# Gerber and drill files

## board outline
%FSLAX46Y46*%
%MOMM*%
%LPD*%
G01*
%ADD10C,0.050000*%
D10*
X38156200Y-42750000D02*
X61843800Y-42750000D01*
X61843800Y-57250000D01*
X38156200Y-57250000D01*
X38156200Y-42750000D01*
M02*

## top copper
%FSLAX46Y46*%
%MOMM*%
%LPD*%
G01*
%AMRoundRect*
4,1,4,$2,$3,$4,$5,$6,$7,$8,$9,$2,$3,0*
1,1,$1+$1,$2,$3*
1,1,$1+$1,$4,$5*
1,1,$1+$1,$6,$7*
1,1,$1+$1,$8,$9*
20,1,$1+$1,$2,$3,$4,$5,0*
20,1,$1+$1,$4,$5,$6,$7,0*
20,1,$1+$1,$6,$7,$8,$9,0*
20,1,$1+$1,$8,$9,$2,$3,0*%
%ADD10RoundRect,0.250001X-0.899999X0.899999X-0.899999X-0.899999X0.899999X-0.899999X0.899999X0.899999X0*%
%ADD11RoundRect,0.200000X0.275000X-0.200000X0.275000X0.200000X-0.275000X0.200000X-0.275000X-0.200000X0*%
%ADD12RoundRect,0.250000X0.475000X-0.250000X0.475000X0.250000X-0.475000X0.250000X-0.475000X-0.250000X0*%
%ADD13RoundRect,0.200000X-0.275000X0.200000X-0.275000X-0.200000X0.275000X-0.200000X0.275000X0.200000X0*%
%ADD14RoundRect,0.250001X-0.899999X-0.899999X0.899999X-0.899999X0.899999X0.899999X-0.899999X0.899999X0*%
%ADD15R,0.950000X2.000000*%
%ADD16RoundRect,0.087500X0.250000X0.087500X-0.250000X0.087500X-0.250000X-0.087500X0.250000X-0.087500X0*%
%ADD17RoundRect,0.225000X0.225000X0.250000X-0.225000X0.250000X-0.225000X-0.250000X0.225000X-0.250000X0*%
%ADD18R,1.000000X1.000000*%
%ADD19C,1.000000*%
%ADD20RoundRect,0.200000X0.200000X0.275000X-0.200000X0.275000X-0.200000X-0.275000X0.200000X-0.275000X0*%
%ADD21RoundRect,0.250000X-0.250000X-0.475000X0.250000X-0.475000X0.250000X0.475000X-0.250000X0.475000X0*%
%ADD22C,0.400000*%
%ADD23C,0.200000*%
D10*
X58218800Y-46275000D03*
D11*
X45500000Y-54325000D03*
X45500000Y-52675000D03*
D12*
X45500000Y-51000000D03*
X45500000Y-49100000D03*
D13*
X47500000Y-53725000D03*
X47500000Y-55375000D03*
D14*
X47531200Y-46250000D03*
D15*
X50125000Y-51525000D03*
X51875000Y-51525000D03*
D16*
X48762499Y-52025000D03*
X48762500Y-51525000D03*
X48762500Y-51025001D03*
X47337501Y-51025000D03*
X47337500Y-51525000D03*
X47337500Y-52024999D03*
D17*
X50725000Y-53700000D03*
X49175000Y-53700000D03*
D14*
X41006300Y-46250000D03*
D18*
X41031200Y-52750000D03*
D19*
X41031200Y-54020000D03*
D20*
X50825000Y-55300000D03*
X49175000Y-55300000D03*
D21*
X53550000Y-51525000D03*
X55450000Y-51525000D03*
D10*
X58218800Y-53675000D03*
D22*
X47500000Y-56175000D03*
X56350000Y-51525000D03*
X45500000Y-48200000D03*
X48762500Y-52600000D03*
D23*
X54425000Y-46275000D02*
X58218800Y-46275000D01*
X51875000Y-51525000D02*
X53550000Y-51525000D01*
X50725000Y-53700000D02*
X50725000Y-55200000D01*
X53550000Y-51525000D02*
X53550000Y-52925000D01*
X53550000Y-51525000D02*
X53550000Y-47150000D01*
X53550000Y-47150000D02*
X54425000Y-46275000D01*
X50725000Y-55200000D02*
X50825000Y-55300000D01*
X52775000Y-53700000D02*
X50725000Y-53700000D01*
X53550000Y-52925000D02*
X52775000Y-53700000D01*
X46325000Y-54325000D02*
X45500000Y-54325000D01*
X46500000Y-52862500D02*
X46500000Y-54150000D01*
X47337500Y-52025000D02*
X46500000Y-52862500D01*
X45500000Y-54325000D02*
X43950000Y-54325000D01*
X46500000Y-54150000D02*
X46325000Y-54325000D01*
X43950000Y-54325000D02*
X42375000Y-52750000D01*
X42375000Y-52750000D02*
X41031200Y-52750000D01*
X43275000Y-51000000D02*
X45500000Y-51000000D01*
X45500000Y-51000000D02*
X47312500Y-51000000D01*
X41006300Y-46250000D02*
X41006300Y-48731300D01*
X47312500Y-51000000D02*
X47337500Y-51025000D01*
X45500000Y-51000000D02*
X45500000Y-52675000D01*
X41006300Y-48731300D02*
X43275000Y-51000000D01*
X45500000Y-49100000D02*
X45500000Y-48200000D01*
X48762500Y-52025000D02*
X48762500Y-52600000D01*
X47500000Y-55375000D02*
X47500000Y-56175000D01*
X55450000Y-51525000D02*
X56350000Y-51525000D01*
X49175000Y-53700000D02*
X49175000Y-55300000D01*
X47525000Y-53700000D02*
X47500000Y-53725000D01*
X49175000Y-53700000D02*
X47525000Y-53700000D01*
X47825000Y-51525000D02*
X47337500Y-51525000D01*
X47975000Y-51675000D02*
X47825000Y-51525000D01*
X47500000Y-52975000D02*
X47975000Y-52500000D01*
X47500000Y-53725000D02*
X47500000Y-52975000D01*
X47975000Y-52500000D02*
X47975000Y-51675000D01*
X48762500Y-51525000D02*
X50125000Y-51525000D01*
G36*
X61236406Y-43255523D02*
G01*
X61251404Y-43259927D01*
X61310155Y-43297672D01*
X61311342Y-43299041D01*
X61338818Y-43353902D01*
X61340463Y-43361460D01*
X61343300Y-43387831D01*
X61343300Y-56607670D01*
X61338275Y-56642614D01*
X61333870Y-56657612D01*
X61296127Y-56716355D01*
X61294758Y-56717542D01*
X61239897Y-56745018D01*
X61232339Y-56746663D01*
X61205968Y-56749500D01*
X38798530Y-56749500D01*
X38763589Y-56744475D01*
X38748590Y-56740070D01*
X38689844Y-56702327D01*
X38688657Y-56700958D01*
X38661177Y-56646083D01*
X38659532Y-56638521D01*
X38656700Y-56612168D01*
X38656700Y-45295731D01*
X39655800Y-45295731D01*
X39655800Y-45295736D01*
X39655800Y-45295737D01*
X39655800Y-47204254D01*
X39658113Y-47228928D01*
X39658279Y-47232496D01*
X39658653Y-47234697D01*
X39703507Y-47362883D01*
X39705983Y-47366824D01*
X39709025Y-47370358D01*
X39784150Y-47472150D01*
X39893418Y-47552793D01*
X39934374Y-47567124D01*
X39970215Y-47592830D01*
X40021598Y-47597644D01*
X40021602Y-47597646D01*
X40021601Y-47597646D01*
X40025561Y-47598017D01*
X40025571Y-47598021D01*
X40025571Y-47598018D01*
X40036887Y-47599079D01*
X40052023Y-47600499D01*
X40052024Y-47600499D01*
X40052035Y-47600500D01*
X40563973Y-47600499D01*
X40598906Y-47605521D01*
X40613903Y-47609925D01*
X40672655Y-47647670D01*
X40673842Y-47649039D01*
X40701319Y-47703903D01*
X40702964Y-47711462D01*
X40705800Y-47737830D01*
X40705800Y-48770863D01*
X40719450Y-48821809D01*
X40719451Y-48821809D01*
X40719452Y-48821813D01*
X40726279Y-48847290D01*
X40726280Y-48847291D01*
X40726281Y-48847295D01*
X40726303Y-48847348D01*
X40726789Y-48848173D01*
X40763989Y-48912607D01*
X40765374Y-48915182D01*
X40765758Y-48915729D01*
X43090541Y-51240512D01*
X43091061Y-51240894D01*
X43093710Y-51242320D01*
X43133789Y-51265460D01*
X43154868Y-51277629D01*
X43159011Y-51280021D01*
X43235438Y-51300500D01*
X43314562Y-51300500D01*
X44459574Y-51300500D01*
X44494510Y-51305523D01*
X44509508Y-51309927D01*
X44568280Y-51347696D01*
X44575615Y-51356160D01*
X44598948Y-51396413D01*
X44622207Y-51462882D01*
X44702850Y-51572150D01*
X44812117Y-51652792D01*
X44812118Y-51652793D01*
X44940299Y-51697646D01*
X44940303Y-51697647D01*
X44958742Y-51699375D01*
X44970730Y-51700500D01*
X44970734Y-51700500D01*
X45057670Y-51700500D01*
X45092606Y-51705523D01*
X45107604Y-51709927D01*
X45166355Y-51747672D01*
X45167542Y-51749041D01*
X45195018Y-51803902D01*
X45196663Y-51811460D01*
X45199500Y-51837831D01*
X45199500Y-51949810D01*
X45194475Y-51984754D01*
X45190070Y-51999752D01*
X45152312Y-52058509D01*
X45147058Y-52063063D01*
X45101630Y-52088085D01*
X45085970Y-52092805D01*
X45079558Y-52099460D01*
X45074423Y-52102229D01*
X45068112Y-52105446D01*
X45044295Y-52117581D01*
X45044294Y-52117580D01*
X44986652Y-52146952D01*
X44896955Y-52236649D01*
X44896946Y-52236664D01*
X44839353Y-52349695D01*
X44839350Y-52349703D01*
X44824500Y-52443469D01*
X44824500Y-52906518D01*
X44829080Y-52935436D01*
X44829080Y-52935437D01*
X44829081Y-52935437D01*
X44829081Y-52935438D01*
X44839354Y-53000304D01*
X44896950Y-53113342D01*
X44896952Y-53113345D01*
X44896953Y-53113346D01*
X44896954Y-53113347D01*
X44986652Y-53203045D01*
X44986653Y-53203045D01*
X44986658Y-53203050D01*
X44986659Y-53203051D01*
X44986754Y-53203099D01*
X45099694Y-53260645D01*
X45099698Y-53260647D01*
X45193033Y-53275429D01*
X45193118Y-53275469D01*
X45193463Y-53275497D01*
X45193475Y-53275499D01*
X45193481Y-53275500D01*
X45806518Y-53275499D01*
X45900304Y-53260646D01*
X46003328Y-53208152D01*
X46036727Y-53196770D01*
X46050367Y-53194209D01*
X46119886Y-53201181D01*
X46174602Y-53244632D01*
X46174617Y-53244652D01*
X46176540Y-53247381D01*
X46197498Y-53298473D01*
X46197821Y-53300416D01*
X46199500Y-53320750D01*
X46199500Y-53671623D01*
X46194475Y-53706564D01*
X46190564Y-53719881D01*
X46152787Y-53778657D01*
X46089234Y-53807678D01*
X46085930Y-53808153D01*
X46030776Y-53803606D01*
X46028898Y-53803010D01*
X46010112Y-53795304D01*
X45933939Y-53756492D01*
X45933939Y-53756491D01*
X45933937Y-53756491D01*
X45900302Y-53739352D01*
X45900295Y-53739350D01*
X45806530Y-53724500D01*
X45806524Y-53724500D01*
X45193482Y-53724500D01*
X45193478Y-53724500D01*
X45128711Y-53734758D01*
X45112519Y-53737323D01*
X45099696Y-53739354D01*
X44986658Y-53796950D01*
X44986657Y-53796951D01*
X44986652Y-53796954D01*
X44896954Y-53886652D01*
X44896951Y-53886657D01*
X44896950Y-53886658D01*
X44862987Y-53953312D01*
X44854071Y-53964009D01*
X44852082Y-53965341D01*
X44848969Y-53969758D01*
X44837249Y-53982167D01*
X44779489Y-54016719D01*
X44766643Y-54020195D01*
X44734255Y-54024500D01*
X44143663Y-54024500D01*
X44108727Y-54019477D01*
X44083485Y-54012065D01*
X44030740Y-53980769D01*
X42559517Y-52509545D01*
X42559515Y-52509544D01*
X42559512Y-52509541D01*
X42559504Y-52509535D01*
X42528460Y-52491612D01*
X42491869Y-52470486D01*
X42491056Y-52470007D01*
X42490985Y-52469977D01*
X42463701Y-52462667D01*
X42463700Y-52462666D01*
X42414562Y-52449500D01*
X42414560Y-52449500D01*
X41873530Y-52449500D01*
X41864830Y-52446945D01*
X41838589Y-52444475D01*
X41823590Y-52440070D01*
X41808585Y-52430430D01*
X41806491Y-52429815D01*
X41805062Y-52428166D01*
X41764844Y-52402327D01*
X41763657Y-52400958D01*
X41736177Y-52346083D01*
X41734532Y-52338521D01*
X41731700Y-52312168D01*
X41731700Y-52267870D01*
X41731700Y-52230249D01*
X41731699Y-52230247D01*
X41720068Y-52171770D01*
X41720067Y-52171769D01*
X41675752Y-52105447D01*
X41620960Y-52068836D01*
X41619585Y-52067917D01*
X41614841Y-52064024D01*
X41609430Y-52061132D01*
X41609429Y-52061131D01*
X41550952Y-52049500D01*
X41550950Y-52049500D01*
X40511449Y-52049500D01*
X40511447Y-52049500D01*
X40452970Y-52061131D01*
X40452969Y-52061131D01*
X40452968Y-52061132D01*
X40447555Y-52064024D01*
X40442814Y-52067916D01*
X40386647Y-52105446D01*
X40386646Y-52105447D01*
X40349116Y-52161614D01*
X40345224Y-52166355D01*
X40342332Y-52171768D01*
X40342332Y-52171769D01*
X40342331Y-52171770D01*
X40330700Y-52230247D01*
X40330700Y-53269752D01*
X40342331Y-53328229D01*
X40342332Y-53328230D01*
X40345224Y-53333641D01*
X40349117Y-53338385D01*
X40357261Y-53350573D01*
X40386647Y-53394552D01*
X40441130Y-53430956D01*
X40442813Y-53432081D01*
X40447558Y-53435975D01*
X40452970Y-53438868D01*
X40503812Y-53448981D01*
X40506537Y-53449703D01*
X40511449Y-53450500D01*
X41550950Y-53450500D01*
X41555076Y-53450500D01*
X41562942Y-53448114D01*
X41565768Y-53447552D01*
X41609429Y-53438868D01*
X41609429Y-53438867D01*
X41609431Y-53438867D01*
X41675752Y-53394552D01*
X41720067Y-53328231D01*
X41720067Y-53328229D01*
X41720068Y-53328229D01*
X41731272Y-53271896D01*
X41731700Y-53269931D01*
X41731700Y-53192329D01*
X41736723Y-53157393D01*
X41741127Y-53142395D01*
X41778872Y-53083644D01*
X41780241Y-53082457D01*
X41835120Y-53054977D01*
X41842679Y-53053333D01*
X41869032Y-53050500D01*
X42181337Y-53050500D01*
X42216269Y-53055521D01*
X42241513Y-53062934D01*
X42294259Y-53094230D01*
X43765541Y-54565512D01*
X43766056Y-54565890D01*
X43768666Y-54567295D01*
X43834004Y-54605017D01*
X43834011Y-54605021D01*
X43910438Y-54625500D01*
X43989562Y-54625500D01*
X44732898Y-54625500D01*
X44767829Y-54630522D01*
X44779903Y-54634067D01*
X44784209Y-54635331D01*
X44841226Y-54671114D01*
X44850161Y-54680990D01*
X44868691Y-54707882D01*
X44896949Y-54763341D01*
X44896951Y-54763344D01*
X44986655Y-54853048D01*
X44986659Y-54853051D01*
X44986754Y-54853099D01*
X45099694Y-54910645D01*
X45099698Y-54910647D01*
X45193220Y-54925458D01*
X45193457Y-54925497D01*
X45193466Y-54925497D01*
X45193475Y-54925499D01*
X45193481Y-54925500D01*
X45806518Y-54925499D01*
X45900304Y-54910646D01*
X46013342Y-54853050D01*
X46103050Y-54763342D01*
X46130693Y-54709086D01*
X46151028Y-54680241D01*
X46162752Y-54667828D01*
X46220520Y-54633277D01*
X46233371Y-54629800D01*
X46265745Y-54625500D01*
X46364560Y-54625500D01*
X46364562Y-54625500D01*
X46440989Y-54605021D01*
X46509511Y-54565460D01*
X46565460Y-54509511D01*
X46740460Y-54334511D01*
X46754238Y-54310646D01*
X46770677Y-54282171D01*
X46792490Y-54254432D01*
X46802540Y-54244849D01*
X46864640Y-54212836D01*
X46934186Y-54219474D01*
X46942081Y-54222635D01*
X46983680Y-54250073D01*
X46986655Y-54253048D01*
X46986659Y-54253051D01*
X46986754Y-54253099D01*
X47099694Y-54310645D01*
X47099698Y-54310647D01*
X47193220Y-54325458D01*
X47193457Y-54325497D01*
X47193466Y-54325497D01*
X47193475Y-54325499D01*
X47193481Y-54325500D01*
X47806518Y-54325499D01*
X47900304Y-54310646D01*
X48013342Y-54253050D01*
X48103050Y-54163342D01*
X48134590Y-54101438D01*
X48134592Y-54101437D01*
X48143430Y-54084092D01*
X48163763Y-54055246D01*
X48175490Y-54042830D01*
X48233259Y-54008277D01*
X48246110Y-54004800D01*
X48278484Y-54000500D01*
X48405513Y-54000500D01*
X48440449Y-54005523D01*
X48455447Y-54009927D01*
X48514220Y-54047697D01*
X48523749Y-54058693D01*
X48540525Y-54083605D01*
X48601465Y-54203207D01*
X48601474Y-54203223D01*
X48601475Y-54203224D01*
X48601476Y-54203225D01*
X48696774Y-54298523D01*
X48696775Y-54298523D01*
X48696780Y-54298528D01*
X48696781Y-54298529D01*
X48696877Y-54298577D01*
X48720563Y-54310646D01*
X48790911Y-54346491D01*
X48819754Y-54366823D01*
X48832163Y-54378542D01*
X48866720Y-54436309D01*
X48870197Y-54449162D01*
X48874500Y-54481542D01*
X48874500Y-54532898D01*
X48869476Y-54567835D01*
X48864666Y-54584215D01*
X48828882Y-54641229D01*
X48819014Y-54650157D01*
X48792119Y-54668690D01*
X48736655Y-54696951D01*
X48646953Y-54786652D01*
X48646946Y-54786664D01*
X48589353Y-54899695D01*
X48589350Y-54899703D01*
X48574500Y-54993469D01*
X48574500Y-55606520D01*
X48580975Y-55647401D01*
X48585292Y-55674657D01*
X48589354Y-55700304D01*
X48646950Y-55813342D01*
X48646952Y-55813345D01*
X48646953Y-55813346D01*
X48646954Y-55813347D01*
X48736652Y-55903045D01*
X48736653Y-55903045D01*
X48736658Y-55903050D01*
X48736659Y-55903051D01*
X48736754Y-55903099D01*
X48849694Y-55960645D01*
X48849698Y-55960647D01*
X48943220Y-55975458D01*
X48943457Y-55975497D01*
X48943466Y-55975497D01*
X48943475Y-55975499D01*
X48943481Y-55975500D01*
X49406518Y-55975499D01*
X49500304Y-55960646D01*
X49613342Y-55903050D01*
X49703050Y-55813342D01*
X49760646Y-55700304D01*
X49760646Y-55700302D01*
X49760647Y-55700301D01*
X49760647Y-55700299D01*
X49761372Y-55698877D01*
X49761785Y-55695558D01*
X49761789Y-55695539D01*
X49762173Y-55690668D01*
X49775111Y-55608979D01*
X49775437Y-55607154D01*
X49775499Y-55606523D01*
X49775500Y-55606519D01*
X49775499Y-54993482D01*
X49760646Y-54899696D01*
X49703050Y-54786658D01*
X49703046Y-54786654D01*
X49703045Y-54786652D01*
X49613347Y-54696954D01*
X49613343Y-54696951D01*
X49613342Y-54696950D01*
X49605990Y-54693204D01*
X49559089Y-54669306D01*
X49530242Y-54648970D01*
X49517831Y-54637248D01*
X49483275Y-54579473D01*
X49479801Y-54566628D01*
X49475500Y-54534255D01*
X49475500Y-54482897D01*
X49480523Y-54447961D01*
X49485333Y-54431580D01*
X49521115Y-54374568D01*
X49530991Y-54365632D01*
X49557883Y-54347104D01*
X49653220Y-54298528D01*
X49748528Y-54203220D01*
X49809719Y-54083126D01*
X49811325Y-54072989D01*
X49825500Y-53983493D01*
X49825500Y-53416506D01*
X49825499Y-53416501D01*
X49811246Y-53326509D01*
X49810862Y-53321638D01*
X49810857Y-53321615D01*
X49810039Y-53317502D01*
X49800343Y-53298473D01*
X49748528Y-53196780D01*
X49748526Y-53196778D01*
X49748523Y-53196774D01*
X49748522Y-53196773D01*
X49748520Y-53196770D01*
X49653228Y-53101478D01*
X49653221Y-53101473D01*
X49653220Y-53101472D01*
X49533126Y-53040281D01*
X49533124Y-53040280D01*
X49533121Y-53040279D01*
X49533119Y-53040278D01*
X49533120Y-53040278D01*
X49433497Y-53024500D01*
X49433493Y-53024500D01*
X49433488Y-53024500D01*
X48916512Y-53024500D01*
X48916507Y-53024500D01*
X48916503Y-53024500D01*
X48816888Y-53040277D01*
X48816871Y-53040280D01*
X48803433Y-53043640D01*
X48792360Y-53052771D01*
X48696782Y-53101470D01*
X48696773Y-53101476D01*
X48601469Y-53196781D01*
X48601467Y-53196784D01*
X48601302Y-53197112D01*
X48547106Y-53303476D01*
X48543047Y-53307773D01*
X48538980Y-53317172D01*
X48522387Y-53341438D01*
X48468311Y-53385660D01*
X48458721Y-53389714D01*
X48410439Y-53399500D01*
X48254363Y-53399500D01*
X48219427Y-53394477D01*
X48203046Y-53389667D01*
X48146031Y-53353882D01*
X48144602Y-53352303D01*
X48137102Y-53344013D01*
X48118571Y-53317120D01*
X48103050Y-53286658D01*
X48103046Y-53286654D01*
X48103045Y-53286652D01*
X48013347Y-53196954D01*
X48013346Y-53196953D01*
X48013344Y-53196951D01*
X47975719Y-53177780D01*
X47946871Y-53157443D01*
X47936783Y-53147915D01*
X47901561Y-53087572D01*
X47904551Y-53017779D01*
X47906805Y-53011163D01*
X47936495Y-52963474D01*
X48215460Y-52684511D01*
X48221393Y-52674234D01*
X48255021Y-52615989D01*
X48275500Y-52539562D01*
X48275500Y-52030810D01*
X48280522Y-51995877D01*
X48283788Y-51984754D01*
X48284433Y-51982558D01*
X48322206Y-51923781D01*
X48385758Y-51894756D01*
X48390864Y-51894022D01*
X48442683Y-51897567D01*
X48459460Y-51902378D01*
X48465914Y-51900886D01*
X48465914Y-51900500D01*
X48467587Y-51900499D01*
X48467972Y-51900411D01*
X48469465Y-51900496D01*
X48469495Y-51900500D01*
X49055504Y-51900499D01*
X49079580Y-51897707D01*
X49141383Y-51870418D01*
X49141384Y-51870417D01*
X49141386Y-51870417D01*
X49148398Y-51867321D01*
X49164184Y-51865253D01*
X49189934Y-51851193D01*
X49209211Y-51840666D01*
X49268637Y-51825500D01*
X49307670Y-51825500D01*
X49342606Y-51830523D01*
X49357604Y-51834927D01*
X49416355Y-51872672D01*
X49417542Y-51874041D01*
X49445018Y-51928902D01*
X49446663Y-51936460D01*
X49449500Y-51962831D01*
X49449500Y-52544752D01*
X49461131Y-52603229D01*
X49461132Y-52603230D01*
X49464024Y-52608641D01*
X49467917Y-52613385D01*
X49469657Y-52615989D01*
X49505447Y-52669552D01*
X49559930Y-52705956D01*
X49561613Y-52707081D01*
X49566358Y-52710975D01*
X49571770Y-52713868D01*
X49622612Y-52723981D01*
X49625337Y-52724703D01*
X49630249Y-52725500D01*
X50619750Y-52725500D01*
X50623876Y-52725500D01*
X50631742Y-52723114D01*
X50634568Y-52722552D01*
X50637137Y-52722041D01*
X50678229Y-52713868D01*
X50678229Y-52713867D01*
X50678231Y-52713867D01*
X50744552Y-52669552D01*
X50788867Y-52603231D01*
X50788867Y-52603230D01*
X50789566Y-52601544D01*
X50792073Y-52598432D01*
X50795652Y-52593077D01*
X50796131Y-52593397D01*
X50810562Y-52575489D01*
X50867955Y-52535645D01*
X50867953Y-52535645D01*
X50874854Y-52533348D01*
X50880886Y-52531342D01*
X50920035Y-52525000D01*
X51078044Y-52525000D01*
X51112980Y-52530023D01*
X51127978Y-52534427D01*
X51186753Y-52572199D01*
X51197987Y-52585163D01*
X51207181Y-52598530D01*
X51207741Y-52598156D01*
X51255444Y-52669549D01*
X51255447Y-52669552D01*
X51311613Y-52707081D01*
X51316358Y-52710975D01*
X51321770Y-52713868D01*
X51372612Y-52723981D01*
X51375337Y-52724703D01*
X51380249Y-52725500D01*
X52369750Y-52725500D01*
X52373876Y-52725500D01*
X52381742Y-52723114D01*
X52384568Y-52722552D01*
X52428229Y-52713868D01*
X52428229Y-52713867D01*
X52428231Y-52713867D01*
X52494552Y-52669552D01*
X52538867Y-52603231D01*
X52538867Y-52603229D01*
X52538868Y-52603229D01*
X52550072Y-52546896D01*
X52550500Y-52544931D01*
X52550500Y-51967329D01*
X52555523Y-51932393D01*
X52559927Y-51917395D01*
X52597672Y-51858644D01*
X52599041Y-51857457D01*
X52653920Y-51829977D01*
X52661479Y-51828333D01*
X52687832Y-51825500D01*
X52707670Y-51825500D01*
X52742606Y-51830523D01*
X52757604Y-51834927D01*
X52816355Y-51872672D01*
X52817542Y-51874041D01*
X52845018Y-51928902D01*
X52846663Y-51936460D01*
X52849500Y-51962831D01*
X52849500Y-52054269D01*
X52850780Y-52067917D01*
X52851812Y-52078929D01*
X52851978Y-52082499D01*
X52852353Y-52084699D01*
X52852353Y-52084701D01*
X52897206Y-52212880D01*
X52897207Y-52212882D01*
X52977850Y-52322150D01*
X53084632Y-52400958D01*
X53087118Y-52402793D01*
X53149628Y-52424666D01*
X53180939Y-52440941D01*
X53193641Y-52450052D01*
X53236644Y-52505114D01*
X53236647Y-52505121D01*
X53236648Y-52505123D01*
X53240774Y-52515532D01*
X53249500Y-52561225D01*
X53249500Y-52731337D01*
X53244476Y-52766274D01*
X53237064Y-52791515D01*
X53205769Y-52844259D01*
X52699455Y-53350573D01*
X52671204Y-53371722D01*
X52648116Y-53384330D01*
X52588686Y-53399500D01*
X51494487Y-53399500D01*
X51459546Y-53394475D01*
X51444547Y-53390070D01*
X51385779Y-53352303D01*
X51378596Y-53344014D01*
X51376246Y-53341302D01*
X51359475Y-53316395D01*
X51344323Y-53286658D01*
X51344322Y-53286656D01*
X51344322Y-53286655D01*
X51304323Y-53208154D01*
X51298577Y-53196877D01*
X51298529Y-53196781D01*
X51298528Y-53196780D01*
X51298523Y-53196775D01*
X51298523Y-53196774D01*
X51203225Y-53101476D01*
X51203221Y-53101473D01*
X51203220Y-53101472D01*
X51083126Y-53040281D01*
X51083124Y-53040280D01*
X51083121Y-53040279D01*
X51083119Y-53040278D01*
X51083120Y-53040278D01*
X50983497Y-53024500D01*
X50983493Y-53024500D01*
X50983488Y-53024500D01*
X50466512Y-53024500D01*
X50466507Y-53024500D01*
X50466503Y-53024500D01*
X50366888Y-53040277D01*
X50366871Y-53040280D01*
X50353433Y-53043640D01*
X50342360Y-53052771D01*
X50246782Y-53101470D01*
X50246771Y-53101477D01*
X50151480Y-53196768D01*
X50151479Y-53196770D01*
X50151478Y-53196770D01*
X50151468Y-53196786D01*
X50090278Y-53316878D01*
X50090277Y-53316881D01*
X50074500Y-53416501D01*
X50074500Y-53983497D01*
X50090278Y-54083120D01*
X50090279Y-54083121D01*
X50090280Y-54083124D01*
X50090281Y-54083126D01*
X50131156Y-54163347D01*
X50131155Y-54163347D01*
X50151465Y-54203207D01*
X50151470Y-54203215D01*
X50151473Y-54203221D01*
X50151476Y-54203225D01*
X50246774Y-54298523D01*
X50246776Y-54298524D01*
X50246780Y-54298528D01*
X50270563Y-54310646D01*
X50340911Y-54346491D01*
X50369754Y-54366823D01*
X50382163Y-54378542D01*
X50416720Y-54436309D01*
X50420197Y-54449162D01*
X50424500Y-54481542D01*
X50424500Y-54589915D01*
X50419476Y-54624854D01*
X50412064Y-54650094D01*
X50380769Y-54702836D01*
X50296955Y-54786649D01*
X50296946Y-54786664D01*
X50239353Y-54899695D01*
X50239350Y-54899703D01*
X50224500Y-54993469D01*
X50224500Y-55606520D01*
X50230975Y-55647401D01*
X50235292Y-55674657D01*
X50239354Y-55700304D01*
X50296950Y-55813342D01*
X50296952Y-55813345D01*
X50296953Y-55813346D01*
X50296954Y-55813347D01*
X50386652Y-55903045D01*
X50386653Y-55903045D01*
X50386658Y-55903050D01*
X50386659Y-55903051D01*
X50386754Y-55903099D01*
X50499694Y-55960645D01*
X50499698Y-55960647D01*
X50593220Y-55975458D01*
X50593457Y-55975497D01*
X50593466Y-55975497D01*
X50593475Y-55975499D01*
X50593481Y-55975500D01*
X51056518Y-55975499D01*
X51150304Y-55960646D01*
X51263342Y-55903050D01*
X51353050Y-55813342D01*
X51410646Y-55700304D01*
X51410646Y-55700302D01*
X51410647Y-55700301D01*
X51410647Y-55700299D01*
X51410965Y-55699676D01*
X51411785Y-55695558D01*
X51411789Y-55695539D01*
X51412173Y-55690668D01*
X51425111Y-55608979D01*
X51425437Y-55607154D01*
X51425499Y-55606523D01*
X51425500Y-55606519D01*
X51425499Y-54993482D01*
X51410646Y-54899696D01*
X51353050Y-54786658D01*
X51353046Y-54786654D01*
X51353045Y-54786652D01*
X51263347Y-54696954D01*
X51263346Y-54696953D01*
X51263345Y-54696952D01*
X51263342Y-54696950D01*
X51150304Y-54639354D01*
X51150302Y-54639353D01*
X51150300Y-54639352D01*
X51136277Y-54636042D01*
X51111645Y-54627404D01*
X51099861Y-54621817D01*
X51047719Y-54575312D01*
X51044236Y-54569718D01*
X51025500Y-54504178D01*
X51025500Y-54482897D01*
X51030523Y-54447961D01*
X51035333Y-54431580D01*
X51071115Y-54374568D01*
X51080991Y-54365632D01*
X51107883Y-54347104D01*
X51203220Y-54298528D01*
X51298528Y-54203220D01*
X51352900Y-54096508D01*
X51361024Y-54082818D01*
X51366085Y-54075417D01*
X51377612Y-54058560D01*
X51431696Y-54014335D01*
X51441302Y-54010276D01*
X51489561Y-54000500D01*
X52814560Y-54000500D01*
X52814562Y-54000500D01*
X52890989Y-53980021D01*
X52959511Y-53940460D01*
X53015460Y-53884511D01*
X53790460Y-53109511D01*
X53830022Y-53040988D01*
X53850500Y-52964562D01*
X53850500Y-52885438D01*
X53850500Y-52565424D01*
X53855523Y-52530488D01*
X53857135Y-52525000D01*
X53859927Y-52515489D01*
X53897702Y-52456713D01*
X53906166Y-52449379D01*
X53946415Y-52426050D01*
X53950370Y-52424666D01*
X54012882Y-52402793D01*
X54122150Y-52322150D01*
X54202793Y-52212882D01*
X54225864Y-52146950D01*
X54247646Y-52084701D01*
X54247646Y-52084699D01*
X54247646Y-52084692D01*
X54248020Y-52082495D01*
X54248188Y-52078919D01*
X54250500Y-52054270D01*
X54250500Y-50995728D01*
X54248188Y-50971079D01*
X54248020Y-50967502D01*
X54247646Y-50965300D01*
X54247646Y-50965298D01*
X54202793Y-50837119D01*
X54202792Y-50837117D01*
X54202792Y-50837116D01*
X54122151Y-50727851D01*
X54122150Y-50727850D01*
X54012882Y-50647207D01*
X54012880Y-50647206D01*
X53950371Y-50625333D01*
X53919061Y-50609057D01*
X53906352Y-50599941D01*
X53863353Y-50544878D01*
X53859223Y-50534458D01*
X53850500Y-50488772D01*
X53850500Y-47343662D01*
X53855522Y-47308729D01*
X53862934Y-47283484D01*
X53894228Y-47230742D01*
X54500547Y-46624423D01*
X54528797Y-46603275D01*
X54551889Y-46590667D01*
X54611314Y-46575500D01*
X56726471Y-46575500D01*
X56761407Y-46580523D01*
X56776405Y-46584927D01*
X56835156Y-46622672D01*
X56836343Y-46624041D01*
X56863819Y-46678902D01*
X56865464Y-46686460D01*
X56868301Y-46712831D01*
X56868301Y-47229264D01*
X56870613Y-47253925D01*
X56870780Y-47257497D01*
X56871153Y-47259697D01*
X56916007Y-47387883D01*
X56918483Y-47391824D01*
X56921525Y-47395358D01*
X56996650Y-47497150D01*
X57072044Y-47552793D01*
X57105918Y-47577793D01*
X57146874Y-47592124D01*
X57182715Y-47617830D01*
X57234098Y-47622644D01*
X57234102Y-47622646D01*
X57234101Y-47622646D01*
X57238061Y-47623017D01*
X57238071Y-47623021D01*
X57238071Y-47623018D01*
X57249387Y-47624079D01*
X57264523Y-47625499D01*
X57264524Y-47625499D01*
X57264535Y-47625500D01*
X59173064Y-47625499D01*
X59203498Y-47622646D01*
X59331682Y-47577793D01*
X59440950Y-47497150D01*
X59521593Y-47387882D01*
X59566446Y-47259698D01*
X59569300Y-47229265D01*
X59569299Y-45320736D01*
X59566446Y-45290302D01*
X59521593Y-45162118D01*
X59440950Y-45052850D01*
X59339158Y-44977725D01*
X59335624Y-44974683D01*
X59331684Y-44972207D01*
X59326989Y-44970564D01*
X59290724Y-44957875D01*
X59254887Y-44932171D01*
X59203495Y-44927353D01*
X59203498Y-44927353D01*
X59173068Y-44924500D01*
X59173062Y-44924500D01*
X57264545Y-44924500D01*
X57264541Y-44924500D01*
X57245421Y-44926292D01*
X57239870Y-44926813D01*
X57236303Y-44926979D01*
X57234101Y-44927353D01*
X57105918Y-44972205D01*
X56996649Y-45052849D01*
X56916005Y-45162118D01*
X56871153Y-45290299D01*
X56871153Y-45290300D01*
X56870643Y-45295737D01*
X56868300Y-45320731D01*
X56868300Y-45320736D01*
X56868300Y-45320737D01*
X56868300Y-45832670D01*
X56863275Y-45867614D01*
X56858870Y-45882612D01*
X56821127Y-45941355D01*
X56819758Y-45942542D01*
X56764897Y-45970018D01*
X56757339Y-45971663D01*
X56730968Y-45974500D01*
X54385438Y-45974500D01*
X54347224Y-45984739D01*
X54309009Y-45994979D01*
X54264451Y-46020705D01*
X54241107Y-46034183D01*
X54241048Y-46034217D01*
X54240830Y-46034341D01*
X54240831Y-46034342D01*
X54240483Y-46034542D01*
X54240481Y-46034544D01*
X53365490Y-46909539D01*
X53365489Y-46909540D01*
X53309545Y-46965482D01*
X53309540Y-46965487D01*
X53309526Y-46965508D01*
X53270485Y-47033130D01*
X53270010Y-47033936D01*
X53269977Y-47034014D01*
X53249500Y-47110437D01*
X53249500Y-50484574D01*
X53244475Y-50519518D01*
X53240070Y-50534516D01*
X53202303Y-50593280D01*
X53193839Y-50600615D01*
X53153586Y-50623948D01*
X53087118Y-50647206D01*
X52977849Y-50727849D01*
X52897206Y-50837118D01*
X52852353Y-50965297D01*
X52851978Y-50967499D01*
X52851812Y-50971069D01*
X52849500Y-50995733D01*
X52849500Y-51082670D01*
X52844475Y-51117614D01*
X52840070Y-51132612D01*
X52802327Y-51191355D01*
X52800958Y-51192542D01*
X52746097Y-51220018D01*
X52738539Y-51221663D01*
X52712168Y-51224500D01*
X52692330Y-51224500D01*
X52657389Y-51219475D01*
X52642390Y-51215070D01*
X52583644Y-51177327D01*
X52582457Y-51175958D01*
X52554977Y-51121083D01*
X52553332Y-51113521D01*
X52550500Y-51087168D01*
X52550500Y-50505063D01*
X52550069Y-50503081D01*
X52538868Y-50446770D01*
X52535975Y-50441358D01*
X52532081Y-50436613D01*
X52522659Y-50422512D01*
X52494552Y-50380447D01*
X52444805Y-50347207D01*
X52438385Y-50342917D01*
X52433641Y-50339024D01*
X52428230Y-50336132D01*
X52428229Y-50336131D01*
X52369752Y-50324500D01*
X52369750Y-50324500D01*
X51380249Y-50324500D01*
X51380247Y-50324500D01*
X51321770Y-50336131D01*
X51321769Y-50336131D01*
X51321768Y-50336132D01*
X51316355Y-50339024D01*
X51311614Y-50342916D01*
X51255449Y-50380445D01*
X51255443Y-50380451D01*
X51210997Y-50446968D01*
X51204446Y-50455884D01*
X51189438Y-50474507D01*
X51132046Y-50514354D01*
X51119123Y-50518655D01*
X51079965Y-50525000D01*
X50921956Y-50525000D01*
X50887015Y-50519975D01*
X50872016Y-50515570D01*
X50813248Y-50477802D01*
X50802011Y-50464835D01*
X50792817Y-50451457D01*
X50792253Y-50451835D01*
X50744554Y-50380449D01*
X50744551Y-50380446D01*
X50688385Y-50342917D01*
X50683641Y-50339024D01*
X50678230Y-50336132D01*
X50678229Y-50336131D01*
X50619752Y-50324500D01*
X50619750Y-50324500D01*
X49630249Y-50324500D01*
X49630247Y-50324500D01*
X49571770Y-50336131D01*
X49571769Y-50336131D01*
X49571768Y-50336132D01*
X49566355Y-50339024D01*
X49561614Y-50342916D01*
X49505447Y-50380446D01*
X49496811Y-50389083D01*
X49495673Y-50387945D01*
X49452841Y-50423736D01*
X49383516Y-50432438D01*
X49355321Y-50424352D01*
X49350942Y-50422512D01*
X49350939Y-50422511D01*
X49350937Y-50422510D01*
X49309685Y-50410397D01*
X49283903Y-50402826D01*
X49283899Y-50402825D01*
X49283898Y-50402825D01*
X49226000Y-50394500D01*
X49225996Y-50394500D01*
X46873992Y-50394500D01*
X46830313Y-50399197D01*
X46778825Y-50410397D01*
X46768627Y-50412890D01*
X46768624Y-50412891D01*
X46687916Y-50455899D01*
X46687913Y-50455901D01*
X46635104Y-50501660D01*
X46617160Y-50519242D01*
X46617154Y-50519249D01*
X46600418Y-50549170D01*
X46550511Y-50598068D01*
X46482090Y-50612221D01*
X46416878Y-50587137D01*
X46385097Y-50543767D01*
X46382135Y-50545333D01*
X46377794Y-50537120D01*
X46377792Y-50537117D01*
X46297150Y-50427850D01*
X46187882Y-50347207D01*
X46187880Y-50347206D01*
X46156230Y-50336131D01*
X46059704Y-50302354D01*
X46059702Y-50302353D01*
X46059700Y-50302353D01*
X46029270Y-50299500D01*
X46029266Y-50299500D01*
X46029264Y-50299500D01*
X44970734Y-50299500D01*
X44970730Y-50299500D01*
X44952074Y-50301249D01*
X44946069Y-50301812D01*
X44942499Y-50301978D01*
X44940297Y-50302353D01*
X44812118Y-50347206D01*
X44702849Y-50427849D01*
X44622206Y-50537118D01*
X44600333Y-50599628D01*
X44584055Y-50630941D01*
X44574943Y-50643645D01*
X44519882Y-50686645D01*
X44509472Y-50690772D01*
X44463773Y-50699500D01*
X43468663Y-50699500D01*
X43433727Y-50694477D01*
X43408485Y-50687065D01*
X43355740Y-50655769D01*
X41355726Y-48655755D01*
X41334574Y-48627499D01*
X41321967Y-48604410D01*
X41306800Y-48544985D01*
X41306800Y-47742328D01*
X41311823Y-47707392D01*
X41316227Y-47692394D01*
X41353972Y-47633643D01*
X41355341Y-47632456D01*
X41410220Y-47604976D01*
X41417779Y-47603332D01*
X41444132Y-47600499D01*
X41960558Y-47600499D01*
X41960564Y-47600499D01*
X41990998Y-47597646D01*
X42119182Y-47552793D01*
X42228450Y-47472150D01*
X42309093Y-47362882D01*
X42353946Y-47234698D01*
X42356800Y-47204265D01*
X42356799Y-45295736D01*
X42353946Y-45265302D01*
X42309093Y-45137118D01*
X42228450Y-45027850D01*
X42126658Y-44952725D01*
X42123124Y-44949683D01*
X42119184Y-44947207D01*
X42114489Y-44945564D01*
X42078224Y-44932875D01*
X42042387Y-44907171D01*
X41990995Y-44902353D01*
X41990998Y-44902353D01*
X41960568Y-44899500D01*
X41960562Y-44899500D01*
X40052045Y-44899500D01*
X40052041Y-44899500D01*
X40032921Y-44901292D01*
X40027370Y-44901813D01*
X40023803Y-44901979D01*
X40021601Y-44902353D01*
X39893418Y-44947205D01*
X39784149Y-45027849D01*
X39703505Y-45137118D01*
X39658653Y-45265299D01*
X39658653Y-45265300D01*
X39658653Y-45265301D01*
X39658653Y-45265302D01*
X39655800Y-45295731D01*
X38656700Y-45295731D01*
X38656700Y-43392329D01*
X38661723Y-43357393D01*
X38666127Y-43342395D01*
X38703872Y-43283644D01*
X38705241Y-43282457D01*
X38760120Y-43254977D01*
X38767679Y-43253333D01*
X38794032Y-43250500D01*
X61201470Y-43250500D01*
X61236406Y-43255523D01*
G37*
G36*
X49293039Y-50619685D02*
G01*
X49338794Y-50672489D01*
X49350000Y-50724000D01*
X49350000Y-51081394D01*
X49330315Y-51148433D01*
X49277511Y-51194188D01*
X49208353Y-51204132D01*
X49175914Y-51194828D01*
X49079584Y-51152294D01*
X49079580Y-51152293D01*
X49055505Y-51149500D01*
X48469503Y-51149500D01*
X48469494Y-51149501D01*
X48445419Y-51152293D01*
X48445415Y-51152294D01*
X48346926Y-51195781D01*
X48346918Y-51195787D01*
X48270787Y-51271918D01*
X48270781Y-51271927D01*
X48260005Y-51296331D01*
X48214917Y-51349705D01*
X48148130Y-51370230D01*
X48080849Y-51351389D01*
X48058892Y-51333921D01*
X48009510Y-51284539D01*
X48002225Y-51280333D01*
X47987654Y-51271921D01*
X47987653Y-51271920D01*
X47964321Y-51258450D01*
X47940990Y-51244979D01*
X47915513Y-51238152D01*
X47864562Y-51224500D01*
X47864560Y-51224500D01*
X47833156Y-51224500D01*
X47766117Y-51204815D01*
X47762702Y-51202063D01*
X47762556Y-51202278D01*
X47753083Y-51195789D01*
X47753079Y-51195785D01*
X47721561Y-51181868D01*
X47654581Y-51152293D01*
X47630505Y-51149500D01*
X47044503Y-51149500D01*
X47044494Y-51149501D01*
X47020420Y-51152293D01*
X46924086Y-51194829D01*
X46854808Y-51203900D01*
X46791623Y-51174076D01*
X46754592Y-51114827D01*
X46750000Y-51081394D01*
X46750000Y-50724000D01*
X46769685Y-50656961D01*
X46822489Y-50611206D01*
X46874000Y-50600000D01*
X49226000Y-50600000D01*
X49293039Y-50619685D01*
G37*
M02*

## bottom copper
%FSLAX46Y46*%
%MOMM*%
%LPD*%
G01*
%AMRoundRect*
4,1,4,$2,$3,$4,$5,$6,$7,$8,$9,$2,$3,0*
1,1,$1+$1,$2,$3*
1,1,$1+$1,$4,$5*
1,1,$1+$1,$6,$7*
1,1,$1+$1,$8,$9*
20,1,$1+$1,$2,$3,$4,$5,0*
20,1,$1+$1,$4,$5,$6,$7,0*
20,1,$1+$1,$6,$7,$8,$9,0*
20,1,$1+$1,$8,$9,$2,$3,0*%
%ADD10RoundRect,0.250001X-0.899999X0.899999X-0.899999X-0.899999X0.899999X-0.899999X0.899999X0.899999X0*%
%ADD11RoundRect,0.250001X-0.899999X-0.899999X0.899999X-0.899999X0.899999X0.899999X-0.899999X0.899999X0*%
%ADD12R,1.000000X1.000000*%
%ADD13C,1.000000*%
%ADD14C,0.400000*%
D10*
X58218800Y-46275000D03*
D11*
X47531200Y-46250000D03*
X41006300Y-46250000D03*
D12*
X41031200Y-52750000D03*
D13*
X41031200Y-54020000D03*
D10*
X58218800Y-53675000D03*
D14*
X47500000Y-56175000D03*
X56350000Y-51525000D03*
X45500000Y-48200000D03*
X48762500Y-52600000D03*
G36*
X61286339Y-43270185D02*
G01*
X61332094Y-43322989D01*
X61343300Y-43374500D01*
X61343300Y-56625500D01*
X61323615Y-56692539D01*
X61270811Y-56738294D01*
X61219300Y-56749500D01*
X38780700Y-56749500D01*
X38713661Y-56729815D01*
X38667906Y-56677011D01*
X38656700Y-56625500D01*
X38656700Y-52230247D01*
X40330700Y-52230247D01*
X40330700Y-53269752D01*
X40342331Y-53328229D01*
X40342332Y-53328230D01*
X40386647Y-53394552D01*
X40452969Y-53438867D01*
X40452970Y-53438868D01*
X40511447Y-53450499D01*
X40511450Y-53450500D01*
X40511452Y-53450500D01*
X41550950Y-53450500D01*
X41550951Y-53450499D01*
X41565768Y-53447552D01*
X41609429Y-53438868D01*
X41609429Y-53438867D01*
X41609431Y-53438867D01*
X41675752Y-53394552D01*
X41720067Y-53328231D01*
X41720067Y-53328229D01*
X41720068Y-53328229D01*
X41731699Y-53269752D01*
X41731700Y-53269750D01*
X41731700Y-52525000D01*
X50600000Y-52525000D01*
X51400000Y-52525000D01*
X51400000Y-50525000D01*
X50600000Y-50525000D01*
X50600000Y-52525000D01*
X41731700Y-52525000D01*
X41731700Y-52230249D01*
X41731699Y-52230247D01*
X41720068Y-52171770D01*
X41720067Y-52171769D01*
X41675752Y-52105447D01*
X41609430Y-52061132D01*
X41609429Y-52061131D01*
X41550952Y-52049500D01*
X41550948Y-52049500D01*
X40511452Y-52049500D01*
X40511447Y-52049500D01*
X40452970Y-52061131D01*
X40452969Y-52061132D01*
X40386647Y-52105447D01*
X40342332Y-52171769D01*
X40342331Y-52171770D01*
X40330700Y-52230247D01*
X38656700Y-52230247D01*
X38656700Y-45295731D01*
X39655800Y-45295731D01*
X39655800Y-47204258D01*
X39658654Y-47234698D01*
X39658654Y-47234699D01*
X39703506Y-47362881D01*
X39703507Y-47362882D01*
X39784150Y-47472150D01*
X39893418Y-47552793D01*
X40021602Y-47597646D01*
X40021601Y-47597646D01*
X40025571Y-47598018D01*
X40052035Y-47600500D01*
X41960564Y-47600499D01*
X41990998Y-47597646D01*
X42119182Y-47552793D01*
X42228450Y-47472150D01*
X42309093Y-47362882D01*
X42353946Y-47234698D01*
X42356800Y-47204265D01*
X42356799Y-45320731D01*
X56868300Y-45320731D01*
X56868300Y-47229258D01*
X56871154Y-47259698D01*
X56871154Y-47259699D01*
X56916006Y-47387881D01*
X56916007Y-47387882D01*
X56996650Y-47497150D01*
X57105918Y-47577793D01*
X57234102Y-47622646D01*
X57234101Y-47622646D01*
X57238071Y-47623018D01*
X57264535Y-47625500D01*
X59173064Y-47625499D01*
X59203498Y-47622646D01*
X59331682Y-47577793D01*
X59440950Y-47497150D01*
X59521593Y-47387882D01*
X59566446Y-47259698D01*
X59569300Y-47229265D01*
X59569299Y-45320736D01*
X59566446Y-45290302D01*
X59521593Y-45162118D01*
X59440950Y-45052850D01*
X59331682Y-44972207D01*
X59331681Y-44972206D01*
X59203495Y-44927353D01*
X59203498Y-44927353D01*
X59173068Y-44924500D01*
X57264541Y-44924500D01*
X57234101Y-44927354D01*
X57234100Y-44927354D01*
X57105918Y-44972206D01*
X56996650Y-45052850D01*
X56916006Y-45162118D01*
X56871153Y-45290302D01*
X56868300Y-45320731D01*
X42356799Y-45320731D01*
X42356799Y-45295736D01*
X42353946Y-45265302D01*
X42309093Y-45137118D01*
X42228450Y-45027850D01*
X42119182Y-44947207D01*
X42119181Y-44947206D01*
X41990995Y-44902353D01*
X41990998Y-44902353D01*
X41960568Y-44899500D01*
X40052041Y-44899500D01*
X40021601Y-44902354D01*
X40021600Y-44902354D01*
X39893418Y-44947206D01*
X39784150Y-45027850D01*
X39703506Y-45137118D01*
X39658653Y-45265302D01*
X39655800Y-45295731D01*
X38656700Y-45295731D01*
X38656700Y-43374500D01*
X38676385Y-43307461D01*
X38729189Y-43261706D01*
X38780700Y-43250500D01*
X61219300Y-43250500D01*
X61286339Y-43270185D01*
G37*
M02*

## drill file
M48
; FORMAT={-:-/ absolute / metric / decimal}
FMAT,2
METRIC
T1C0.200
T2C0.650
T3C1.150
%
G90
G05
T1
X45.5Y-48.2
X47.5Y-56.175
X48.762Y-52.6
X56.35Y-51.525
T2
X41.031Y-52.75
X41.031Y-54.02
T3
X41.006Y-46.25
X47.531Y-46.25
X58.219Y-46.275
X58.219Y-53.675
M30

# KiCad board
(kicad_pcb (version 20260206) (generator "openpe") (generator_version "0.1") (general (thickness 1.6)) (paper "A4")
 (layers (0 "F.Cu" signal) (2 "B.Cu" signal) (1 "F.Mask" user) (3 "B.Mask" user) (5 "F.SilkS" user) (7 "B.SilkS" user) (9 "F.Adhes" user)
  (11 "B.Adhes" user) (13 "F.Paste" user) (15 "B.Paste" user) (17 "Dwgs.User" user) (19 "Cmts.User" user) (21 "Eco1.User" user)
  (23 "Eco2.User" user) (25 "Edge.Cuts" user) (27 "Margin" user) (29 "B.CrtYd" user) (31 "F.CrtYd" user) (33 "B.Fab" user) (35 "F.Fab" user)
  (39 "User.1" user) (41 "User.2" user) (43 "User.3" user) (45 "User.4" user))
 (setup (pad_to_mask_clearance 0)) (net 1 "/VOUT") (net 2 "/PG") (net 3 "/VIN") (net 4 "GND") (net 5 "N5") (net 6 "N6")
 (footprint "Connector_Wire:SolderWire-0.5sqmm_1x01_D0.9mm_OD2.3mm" (layer "F.Cu") (at 58.2188 46.275 -90)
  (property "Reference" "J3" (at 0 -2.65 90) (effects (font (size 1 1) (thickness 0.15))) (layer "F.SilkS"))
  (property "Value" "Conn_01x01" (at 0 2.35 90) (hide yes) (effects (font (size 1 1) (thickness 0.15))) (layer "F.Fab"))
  (pad "1" thru_hole roundrect (at 0 0 -90) (size 2.3 2.3) (drill 1.15) (layers "*.Cu" "*.Mask") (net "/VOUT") (roundrect_rratio 0.108696)
   (remove_unused_layers no)))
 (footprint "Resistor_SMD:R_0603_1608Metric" (layer "F.Cu") (at 45.5 53.5 90)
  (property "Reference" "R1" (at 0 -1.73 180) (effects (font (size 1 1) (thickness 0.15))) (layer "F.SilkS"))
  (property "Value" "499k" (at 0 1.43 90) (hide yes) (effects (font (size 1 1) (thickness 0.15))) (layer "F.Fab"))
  (pad "1" smd roundrect (at -0.825 0 90) (size 0.8 0.95) (layers "F.Cu" "F.Mask" "F.Paste") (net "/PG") (roundrect_rratio 0.25))
  (pad "2" smd roundrect (at 0.825 0 90) (size 0.8 0.95) (layers "F.Cu" "F.Mask" "F.Paste") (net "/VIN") (roundrect_rratio 0.25)))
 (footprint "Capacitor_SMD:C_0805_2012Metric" (layer "F.Cu") (at 45.5 50.05 90)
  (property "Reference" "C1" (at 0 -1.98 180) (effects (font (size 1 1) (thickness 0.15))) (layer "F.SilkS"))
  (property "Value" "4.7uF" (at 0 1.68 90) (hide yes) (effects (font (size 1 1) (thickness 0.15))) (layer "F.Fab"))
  (pad "1" smd roundrect (at -0.95 0 90) (size 1 1.45) (layers "F.Cu" "F.Mask" "F.Paste") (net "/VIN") (roundrect_rratio 0.25))
  (pad "2" smd roundrect (at 0.95 0 90) (size 1 1.45) (layers "F.Cu" "F.Mask" "F.Paste") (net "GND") (roundrect_rratio 0.25)))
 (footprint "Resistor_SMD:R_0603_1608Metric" (layer "F.Cu") (at 47.5 54.55 -90)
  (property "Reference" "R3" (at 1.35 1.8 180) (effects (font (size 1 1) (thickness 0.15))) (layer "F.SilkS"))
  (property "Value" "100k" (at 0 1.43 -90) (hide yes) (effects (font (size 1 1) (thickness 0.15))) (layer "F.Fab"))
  (pad "1" smd roundrect (at -0.825 0 -90) (size 0.8 0.95) (layers "F.Cu" "F.Mask" "F.Paste") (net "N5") (roundrect_rratio 0.25))
  (pad "2" smd roundrect (at 0.825 0 -90) (size 0.8 0.95) (layers "F.Cu" "F.Mask" "F.Paste") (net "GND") (roundrect_rratio 0.25)))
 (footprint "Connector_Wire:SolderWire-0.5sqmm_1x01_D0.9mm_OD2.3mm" (layer "F.Cu") (at 47.5312 46.25 0)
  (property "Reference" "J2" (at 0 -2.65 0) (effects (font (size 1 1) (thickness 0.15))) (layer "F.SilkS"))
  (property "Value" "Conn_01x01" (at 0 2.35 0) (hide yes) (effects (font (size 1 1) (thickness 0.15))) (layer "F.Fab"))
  (pad "1" thru_hole roundrect (at 0 0 0) (size 2.3 2.3) (drill 1.15) (layers "*.Cu" "*.Mask") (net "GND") (roundrect_rratio 0.108696)
   (remove_unused_layers no)))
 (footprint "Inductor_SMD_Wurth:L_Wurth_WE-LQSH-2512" (layer "F.Cu") (at 51 51.525 0)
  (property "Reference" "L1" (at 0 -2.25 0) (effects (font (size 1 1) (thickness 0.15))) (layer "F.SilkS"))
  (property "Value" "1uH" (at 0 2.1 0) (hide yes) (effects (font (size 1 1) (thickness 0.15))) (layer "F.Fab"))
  (pad "1" smd rect (at -0.875 0 0) (size 0.95 2) (layers "F.Cu" "F.Mask" "F.Paste") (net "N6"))
  (pad "2" smd rect (at 0.875 0 0) (size 0.95 2) (layers "F.Cu" "F.Mask" "F.Paste") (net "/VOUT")))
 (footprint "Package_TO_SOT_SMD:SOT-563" (layer "F.Cu") (at 48.05 51.525 180)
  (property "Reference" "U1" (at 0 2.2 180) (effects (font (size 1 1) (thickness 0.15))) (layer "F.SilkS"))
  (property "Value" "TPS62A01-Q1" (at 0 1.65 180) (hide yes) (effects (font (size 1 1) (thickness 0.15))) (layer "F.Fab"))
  (pad "1" smd roundrect (at -0.712499 -0.5 180) (size 0.675 0.35) (layers "F.Cu" "F.Mask" "F.Paste") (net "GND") (roundrect_rratio 0.25))
  (pad "2" smd roundrect (at -0.7125 0 180) (size 0.675 0.35) (layers "F.Cu" "F.Mask" "F.Paste") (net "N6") (roundrect_rratio 0.25))
  (pad "3" smd roundrect (at -0.7125 0.499999 180) (size 0.675 0.35) (layers "F.Cu" "F.Mask" "F.Paste") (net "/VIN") (roundrect_rratio 0.25))
  (pad "4" smd roundrect (at 0.712499 0.5 180) (size 0.675 0.35) (layers "F.Cu" "F.Mask" "F.Paste") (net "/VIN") (roundrect_rratio 0.25))
  (pad "5" smd roundrect (at 0.7125 0 180) (size 0.675 0.35) (layers "F.Cu" "F.Mask" "F.Paste") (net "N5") (roundrect_rratio 0.25))
  (pad "6" smd roundrect (at 0.7125 -0.499999 180) (size 0.675 0.35) (layers "F.Cu" "F.Mask" "F.Paste") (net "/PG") (roundrect_rratio 0.25)))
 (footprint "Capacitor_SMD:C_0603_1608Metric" (layer "F.Cu") (at 49.95 53.7 180)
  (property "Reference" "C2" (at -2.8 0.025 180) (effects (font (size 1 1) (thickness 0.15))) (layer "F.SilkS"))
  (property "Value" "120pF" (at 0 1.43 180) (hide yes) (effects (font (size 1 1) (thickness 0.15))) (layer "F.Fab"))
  (pad "1" smd roundrect (at -0.775 0 180) (size 0.9 0.95) (layers "F.Cu" "F.Mask" "F.Paste") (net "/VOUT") (roundrect_rratio 0.25))
  (pad "2" smd roundrect (at 0.775 0 180) (size 0.9 0.95) (layers "F.Cu" "F.Mask" "F.Paste") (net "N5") (roundrect_rratio 0.25)))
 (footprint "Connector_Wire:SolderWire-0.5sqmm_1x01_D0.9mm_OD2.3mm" (layer "F.Cu") (at 41.0063 46.25 0)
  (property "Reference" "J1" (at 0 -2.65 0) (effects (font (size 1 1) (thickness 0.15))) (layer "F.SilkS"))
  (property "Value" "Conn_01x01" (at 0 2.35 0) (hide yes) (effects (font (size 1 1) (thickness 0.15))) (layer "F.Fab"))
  (pad "1" thru_hole roundrect (at 0 0 0) (size 2.3 2.3) (drill 1.15) (layers "*.Cu" "*.Mask") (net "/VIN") (roundrect_rratio 0.108696)
   (remove_unused_layers no)))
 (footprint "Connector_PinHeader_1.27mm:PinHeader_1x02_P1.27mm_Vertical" (layer "F.Cu") (at 41.0312 53.385 0)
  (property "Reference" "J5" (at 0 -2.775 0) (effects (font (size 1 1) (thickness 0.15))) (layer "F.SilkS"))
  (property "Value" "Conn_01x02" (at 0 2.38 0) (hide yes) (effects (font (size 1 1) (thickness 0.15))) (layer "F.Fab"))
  (pad "1" thru_hole rect (at 0 -0.635 0) (size 1 1) (drill 0.65) (layers "*.Cu" "*.Mask") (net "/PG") (remove_unused_layers no))
  (pad "2" thru_hole circle (at 0 0.635 0) (size 1 1) (drill 0.65) (layers "*.Cu" "*.Mask") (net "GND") (remove_unused_layers no)))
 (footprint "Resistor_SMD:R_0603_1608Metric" (layer "F.Cu") (at 50 55.3 180)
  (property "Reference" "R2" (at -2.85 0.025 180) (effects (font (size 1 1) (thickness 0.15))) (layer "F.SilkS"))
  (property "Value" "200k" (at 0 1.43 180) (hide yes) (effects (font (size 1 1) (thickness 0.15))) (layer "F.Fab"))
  (pad "1" smd roundrect (at -0.825 0 180) (size 0.8 0.95) (layers "F.Cu" "F.Mask" "F.Paste") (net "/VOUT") (roundrect_rratio 0.25))
  (pad "2" smd roundrect (at 0.825 0 180) (size 0.8 0.95) (layers "F.Cu" "F.Mask" "F.Paste") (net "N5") (roundrect_rratio 0.25)))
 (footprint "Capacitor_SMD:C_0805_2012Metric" (layer "F.Cu") (at 54.5 51.525 0)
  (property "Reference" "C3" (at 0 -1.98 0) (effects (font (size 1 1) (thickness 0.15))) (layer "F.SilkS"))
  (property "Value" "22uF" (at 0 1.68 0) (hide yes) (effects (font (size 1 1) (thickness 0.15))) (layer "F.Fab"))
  (pad "1" smd roundrect (at -0.95 0 0) (size 1 1.45) (layers "F.Cu" "F.Mask" "F.Paste") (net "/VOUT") (roundrect_rratio 0.25))
  (pad "2" smd roundrect (at 0.95 0 0) (size 1 1.45) (layers "F.Cu" "F.Mask" "F.Paste") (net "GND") (roundrect_rratio 0.25)))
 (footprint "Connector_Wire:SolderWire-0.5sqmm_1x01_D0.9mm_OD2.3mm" (layer "F.Cu") (at 58.2188 53.675 -90)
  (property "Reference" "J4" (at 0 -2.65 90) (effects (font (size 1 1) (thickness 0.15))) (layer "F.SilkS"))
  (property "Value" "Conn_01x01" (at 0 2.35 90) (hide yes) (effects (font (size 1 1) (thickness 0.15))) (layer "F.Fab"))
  (pad "1" thru_hole roundrect (at 0 0 -90) (size 2.3 2.3) (drill 1.15) (layers "*.Cu" "*.Mask") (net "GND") (roundrect_rratio 0.108696)
   (remove_unused_layers no)))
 (gr_poly
  (pts (xy 38.1562 42.75) (xy 61.8438 42.75) (xy 61.8438 57.25) (xy 38.1562 57.25)) (stroke (width 0.05) (type solid)) (fill no)
  (layer "Edge.Cuts"))
 (segment (start 54.425 46.275) (end 58.2188 46.275) (width 0.2) (layer "F.Cu") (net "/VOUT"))
 (segment (start 51.875 51.525) (end 53.55 51.525) (width 0.2) (layer "F.Cu") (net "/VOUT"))
 (segment (start 50.725 53.7) (end 50.725 55.2) (width 0.2) (layer "F.Cu") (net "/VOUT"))
 (segment (start 53.55 51.525) (end 53.55 52.925) (width 0.2) (layer "F.Cu") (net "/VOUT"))
 (segment (start 53.55 51.525) (end 53.55 47.15) (width 0.2) (layer "F.Cu") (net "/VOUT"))
 (segment (start 53.55 47.15) (end 54.425 46.275) (width 0.2) (layer "F.Cu") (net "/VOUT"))
 (segment (start 50.725 55.2) (end 50.825 55.3) (width 0.2) (layer "F.Cu") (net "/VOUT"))
 (segment (start 52.775 53.7) (end 50.725 53.7) (width 0.2) (layer "F.Cu") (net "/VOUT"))
 (segment (start 53.55 52.925) (end 52.775 53.7) (width 0.2) (layer "F.Cu") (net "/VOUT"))
 (segment (start 46.325 54.325) (end 45.5 54.325) (width 0.2) (layer "F.Cu") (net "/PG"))
 (segment (start 46.5 52.8625) (end 46.5 54.15) (width 0.2) (layer "F.Cu") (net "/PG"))
 (segment (start 47.3375 52.025) (end 46.5 52.8625) (width 0.2) (layer "F.Cu") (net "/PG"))
 (segment (start 45.5 54.325) (end 43.95 54.325) (width 0.2) (layer "F.Cu") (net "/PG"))
 (segment (start 46.5 54.15) (end 46.325 54.325) (width 0.2) (layer "F.Cu") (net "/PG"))
 (segment (start 43.95 54.325) (end 42.375 52.75) (width 0.2) (layer "F.Cu") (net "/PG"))
 (segment (start 42.375 52.75) (end 41.0312 52.75) (width 0.2) (layer "F.Cu") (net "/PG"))
 (segment (start 43.275 51) (end 45.5 51) (width 0.2) (layer "F.Cu") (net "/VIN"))
 (segment (start 45.5 51) (end 47.3125 51) (width 0.2) (layer "F.Cu") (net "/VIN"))
 (segment (start 41.0063 46.25) (end 41.0063 48.7313) (width 0.2) (layer "F.Cu") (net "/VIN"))
 (segment (start 47.3125 51) (end 47.3375 51.025) (width 0.2) (layer "F.Cu") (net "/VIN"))
 (segment (start 45.5 51) (end 45.5 52.675) (width 0.2) (layer "F.Cu") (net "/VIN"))
 (segment (start 41.0063 48.7313) (end 43.275 51) (width 0.2) (layer "F.Cu") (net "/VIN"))
 (segment (start 45.5 49.1) (end 45.5 48.2) (width 0.2) (layer "F.Cu") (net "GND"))
 (segment (start 48.7625 52.025) (end 48.7625 52.6) (width 0.2) (layer "F.Cu") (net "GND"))
 (segment (start 47.5 55.375) (end 47.5 56.175) (width 0.2) (layer "F.Cu") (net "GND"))
 (segment (start 55.45 51.525) (end 56.35 51.525) (width 0.2) (layer "F.Cu") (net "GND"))
 (segment (start 49.175 53.7) (end 49.175 55.3) (width 0.2) (layer "F.Cu") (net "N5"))
 (segment (start 47.525 53.7) (end 47.5 53.725) (width 0.2) (layer "F.Cu") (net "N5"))
 (segment (start 49.175 53.7) (end 47.525 53.7) (width 0.2) (layer "F.Cu") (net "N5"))
 (segment (start 47.825 51.525) (end 47.3375 51.525) (width 0.2) (layer "F.Cu") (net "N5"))
 (segment (start 47.975 51.675) (end 47.825 51.525) (width 0.2) (layer "F.Cu") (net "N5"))
 (segment (start 47.5 52.975) (end 47.975 52.5) (width 0.2) (layer "F.Cu") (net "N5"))
 (segment (start 47.5 53.725) (end 47.5 52.975) (width 0.2) (layer "F.Cu") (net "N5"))
 (segment (start 47.975 52.5) (end 47.975 51.675) (width 0.2) (layer "F.Cu") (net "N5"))
 (segment (start 48.7625 51.525) (end 50.125 51.525) (width 0.2) (layer "F.Cu") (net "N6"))
 (via (at 47.5 56.175) (size 0.4) (drill 0.2) (layers "F.Cu" "B.Cu") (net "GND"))
 (via (at 56.35 51.525) (size 0.4) (drill 0.2) (layers "F.Cu" "B.Cu") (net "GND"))
 (via (at 45.5 48.2) (size 0.4) (drill 0.2) (layers "F.Cu" "B.Cu") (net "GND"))
 (via (at 48.7625 52.6) (size 0.4) (drill 0.2) (layers "F.Cu" "B.Cu") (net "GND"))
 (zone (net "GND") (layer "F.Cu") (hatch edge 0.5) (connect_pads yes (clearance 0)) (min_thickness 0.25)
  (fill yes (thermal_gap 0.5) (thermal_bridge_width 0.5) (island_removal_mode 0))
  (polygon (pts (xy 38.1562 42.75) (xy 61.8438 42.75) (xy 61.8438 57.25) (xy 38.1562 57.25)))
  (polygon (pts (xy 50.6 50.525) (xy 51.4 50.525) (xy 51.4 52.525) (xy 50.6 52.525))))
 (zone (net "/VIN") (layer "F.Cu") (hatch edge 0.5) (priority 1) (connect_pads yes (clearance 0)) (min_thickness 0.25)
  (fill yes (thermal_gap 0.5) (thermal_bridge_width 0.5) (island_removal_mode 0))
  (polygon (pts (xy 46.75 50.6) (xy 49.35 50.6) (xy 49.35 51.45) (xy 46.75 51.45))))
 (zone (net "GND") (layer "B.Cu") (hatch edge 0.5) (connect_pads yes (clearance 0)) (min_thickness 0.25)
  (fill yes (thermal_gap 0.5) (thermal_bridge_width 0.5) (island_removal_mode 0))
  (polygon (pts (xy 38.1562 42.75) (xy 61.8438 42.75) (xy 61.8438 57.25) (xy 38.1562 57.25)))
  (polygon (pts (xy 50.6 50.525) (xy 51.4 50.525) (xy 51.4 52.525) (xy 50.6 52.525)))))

